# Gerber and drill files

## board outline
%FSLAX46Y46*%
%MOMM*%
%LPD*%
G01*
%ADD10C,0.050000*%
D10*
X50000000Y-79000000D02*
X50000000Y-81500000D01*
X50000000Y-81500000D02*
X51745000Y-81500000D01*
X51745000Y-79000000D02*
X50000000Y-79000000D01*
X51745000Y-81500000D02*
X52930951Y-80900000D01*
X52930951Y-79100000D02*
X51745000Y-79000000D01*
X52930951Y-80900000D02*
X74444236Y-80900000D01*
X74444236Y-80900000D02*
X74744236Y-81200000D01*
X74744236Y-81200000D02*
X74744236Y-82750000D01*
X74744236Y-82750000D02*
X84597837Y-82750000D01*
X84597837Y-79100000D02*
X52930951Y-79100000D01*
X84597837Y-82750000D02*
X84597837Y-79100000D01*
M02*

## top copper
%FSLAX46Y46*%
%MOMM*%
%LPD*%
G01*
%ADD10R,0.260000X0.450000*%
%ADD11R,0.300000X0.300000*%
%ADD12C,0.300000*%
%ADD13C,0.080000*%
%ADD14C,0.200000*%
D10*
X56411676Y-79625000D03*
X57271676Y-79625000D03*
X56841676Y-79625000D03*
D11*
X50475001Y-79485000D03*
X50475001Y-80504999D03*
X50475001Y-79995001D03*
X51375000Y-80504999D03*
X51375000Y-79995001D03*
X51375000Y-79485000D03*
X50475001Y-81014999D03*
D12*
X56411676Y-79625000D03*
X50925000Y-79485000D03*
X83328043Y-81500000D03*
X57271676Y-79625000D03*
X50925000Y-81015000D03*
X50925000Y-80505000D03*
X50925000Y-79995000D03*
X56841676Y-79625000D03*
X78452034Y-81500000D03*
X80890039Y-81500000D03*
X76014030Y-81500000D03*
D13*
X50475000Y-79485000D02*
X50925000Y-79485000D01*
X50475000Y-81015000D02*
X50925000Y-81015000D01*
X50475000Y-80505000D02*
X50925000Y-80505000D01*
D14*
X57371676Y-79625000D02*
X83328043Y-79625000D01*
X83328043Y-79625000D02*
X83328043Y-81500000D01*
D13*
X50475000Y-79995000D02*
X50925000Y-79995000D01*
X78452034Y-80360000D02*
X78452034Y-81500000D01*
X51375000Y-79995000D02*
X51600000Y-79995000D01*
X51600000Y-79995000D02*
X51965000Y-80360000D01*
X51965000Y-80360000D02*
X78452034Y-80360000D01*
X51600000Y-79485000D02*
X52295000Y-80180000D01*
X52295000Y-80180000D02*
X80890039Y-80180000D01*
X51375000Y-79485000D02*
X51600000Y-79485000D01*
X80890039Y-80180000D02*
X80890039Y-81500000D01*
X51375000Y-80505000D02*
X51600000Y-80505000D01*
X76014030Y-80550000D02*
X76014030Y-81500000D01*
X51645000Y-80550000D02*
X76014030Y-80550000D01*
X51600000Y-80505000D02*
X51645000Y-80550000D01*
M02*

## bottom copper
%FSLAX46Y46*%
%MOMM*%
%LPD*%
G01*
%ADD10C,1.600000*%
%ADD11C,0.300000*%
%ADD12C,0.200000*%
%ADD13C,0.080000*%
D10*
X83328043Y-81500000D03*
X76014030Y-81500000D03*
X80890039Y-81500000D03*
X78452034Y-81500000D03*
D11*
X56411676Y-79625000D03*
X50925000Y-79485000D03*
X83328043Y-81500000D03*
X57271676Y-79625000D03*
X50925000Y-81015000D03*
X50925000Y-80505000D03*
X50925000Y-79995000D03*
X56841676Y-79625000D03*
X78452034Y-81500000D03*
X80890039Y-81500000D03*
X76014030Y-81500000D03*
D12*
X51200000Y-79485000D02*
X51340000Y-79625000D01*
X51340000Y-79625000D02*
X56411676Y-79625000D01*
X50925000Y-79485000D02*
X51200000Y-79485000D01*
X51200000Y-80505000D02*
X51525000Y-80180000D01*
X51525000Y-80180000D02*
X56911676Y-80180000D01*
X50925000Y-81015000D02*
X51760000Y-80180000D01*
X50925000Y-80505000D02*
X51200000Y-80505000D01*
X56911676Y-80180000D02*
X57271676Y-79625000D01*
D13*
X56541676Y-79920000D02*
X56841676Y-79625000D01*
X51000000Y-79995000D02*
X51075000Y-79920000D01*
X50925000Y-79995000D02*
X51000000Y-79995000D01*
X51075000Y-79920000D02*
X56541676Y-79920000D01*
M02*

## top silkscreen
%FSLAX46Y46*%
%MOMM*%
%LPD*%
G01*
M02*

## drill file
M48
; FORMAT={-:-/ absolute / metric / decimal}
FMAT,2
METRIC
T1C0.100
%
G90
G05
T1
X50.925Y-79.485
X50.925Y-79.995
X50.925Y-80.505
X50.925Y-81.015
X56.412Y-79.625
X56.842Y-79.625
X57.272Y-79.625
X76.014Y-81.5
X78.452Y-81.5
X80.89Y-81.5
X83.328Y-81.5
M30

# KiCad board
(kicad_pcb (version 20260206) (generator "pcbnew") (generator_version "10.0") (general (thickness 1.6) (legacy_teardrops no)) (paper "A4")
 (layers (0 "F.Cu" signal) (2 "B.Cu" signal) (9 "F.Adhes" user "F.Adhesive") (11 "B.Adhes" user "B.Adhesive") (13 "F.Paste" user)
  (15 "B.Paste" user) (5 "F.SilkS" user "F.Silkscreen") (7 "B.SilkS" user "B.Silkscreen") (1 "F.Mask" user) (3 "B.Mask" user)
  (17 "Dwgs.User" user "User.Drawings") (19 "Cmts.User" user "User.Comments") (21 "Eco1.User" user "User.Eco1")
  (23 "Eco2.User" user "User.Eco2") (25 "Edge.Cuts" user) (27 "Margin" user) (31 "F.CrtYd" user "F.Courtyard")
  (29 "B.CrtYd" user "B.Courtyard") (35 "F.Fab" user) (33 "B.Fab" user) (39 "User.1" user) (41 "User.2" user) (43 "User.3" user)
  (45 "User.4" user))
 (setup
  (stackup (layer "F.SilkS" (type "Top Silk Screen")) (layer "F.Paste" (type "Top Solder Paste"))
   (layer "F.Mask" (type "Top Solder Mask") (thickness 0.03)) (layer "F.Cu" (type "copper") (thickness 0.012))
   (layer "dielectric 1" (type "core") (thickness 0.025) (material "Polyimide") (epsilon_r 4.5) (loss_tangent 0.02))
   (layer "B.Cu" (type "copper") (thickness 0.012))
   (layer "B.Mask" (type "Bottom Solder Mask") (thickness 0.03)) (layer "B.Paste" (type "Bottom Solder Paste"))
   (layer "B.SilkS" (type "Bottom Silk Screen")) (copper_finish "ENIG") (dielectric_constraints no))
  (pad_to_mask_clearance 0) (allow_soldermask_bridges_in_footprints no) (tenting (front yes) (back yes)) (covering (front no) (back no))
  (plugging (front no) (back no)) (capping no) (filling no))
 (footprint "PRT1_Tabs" (layer "F.Cu") (at 56.841676 79.625)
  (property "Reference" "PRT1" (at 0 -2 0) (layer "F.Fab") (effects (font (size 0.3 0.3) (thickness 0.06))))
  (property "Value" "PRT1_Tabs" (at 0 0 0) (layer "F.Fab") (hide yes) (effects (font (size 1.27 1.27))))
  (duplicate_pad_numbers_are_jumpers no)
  (pad "1" smd rect (at -0.43 0) (size 0.26 0.45) (layers "F.Cu" "F.Mask") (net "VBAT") (solder_mask_margin 0.05) (thermal_bridge_angle 45))
  (pad "2" smd rect (at 0.43 0) (size 0.26 0.45) (layers "F.Cu" "F.Mask") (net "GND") (solder_mask_margin 0.05) (thermal_bridge_angle 45))
  (pad "3" smd rect (at 0 0) (size 0.26 0.45) (layers "F.Cu" "F.Mask") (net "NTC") (solder_mask_margin 0.05) (thermal_bridge_angle 45)))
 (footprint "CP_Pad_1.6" (layer "F.Cu") (at 83.328043 81.5)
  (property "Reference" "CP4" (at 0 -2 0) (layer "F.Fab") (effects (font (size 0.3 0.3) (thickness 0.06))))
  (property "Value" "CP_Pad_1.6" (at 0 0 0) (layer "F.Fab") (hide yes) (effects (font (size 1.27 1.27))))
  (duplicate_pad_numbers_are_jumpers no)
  (pad "1" smd circle (at 0 0) (size 1.6 1.6) (layers "B.Cu" "B.Mask") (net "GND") (solder_mask_margin 0.1)))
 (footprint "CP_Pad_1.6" (layer "F.Cu") (at 76.01403 81.5)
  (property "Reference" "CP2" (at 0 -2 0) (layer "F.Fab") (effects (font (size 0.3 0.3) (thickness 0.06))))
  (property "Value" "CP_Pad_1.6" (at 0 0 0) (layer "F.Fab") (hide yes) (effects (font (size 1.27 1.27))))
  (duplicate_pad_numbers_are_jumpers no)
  (pad "1" smd circle (at 0 0) (size 1.6 1.6) (layers "B.Cu" "B.Mask") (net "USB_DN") (solder_mask_margin 0.1)))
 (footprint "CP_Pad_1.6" (layer "F.Cu") (at 80.890039 81.5)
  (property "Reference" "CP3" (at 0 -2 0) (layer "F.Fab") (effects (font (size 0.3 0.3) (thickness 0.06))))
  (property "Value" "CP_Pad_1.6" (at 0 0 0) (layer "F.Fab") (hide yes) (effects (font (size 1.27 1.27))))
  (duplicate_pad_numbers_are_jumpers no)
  (pad "1" smd circle (at 0 0) (size 1.6 1.6) (layers "B.Cu" "B.Mask") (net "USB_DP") (solder_mask_margin 0.1)))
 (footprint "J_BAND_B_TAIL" (layer "F.Cu") (at 50.9 80.25)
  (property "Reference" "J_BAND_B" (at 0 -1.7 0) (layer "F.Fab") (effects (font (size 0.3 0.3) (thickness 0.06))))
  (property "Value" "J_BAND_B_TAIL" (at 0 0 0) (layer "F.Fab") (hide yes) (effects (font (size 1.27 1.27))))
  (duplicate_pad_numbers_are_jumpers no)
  (pad "1" smd rect (at -0.424999 -0.765) (size 0.3 0.3) (layers "F.Cu" "F.Mask") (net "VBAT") (solder_mask_margin 0.05)
   (thermal_bridge_angle 45))
  (pad "2" smd rect (at -0.424999 0.254999) (size 0.3 0.3) (layers "F.Cu" "F.Mask") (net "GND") (solder_mask_margin 0.05)
   (thermal_bridge_angle 45))
  (pad "3" smd rect (at -0.424999 -0.254999) (size 0.3 0.3) (layers "F.Cu" "F.Mask") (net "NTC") (solder_mask_margin 0.05)
   (thermal_bridge_angle 45))
  (pad "4" smd rect (at 0.475 0.254999) (size 0.3 0.3) (layers "F.Cu" "F.Mask") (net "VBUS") (solder_mask_margin 0.05)
   (thermal_bridge_angle 45))
  (pad "5" smd rect (at 0.475 -0.254999) (size 0.3 0.3) (layers "F.Cu" "F.Mask") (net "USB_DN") (solder_mask_margin 0.05)
   (thermal_bridge_angle 45))
  (pad "6" smd rect (at 0.475 -0.765) (size 0.3 0.3) (layers "F.Cu" "F.Mask") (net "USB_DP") (solder_mask_margin 0.05)
   (thermal_bridge_angle 45))
  (pad "7" smd rect (at -0.424999 0.764999) (size 0.3 0.3) (layers "F.Cu" "F.Mask") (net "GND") (solder_mask_margin 0.05)
   (thermal_bridge_angle 45)))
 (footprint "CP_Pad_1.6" (layer "F.Cu") (at 78.452034 81.5)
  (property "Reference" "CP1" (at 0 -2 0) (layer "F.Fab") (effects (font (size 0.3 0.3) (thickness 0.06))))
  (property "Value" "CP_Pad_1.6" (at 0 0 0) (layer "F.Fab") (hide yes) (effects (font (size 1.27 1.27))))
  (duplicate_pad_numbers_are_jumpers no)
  (pad "1" smd circle (at 0 0) (size 1.6 1.6) (layers "B.Cu" "B.Mask") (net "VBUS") (solder_mask_margin 0.1)))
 (gr_line (start 50 79) (end 50 81.5) (stroke (width 0.05) (type default)) (layer "Edge.Cuts"))
 (gr_line (start 50 81.5) (end 51.745 81.5) (stroke (width 0.05) (type default)) (layer "Edge.Cuts"))
 (gr_line (start 51.745 79) (end 50 79) (stroke (width 0.05) (type default)) (layer "Edge.Cuts"))
 (gr_line (start 51.745 81.5) (end 52.930951 80.9) (stroke (width 0.05) (type default)) (layer "Edge.Cuts"))
 (gr_line (start 52.930951 79.1) (end 51.745 79) (stroke (width 0.05) (type default)) (layer "Edge.Cuts"))
 (gr_line (start 52.930951 80.9) (end 74.444236 80.9) (stroke (width 0.05) (type default)) (layer "Edge.Cuts"))
 (gr_line (start 74.444236 80.9) (end 74.744236 81.2) (stroke (width 0.05) (type default)) (layer "Edge.Cuts"))
 (gr_line (start 74.744236 81.2) (end 74.744236 82.75) (stroke (width 0.05) (type default)) (layer "Edge.Cuts"))
 (gr_line (start 74.744236 82.75) (end 84.597837 82.75) (stroke (width 0.05) (type default)) (layer "Edge.Cuts"))
 (gr_line (start 84.597837 79.1) (end 52.930951 79.1) (stroke (width 0.05) (type default)) (layer "Edge.Cuts"))
 (gr_line (start 84.597837 82.75) (end 84.597837 79.1) (stroke (width 0.05) (type default)) (layer "Edge.Cuts"))
 (segment (start 50.475 79.485) (end 50.925 79.485) (width 0.08) (layer "F.Cu") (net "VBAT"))
 (via (at 56.411676 79.625) (size 0.3) (drill 0.1) (layers "F.Cu" "B.Cu") (tenting (front yes) (back yes)) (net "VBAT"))
 (via (at 50.925 79.485) (size 0.3) (drill 0.1) (layers "F.Cu" "B.Cu") (tenting (front yes) (back yes)) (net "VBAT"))
 (segment (start 51.2 79.485) (end 51.34 79.625) (width 0.2) (layer "B.Cu") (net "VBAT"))
 (segment (start 51.34 79.625) (end 56.411676 79.625) (width 0.2) (layer "B.Cu") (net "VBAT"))
 (segment (start 50.925 79.485) (end 51.2 79.485) (width 0.2) (layer "B.Cu") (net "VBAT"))
 (segment (start 50.475 81.015) (end 50.925 81.015) (width 0.08) (layer "F.Cu") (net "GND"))
 (segment (start 50.475 80.505) (end 50.925 80.505) (width 0.08) (layer "F.Cu") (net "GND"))
 (segment (start 57.371676 79.625) (end 83.328043 79.625) (width 0.2) (layer "F.Cu") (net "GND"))
 (segment (start 83.328043 79.625) (end 83.328043 81.5) (width 0.2) (layer "F.Cu") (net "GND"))
 (via (at 83.328043 81.5) (size 0.3) (drill 0.1) (layers "F.Cu" "B.Cu") (tenting (front yes) (back yes)) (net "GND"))
 (via (at 57.271676 79.625) (size 0.3) (drill 0.1) (layers "F.Cu" "B.Cu") (tenting (front yes) (back yes)) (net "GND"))
 (via (at 50.925 81.015) (size 0.3) (drill 0.1) (layers "F.Cu" "B.Cu") (tenting (front yes) (back yes)) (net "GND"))
 (via (at 50.925 80.505) (size 0.3) (drill 0.1) (layers "F.Cu" "B.Cu") (tenting (front yes) (back yes)) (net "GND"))
 (segment (start 51.2 80.505) (end 51.525 80.18) (width 0.2) (layer "B.Cu") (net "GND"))
 (segment (start 51.525 80.18) (end 56.911676 80.18) (width 0.2) (layer "B.Cu") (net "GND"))
 (segment (start 50.925 81.015) (end 51.76 80.18) (width 0.2) (layer "B.Cu") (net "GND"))
 (segment (start 50.925 80.505) (end 51.2 80.505) (width 0.2) (layer "B.Cu") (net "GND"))
 (segment (start 56.911676 80.18) (end 57.271676 79.625) (width 0.2) (layer "B.Cu") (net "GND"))
 (segment (start 50.475 79.995) (end 50.925 79.995) (width 0.08) (layer "F.Cu") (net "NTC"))
 (via (at 50.925 79.995) (size 0.3) (drill 0.1) (layers "F.Cu" "B.Cu") (tenting (front yes) (back yes)) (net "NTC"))
 (via (at 56.841676 79.625) (size 0.3) (drill 0.1) (layers "F.Cu" "B.Cu") (tenting (front yes) (back yes)) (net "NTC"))
 (segment (start 56.541676 79.92) (end 56.841676 79.625) (width 0.08) (layer "B.Cu") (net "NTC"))
 (segment (start 51 79.995) (end 51.075 79.92) (width 0.08) (layer "B.Cu") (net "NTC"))
 (segment (start 50.925 79.995) (end 51 79.995) (width 0.08) (layer "B.Cu") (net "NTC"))
 (segment (start 51.075 79.92) (end 56.541676 79.92) (width 0.08) (layer "B.Cu") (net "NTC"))
 (segment (start 78.452034 80.36) (end 78.452034 81.5) (width 0.08) (layer "F.Cu") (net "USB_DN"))
 (segment (start 51.375 79.995) (end 51.6 79.995) (width 0.08) (layer "F.Cu") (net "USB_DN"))
 (segment (start 51.6 79.995) (end 51.965 80.36) (width 0.08) (layer "F.Cu") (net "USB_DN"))
 (segment (start 51.965 80.36) (end 78.452034 80.36) (width 0.08) (layer "F.Cu") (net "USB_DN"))
 (via (at 78.452034 81.5) (size 0.3) (drill 0.1) (layers "F.Cu" "B.Cu") (tenting (front yes) (back yes)) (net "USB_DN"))
 (segment (start 51.6 79.485) (end 52.295 80.18) (width 0.08) (layer "F.Cu") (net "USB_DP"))
 (segment (start 52.295 80.18) (end 80.890039 80.18) (width 0.08) (layer "F.Cu") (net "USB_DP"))
 (segment (start 51.375 79.485) (end 51.6 79.485) (width 0.08) (layer "F.Cu") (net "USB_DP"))
 (segment (start 80.890039 80.18) (end 80.890039 81.5) (width 0.08) (layer "F.Cu") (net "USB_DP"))
 (via (at 80.890039 81.5) (size 0.3) (drill 0.1) (layers "F.Cu" "B.Cu") (tenting (front yes) (back yes)) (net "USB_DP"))
 (segment (start 51.375 80.505) (end 51.6 80.505) (width 0.08) (layer "F.Cu") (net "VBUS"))
 (segment (start 76.01403 80.55) (end 76.01403 81.5) (width 0.08) (layer "F.Cu") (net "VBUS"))
 (segment (start 51.645 80.55) (end 76.01403 80.55) (width 0.08) (layer "F.Cu") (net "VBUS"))
 (segment (start 51.6 80.505) (end 51.645 80.55) (width 0.08) (layer "F.Cu") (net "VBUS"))
 (via (at 76.01403 81.5) (size 0.3) (drill 0.1) (layers "F.Cu" "B.Cu") (tenting (front yes) (back yes)) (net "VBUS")))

